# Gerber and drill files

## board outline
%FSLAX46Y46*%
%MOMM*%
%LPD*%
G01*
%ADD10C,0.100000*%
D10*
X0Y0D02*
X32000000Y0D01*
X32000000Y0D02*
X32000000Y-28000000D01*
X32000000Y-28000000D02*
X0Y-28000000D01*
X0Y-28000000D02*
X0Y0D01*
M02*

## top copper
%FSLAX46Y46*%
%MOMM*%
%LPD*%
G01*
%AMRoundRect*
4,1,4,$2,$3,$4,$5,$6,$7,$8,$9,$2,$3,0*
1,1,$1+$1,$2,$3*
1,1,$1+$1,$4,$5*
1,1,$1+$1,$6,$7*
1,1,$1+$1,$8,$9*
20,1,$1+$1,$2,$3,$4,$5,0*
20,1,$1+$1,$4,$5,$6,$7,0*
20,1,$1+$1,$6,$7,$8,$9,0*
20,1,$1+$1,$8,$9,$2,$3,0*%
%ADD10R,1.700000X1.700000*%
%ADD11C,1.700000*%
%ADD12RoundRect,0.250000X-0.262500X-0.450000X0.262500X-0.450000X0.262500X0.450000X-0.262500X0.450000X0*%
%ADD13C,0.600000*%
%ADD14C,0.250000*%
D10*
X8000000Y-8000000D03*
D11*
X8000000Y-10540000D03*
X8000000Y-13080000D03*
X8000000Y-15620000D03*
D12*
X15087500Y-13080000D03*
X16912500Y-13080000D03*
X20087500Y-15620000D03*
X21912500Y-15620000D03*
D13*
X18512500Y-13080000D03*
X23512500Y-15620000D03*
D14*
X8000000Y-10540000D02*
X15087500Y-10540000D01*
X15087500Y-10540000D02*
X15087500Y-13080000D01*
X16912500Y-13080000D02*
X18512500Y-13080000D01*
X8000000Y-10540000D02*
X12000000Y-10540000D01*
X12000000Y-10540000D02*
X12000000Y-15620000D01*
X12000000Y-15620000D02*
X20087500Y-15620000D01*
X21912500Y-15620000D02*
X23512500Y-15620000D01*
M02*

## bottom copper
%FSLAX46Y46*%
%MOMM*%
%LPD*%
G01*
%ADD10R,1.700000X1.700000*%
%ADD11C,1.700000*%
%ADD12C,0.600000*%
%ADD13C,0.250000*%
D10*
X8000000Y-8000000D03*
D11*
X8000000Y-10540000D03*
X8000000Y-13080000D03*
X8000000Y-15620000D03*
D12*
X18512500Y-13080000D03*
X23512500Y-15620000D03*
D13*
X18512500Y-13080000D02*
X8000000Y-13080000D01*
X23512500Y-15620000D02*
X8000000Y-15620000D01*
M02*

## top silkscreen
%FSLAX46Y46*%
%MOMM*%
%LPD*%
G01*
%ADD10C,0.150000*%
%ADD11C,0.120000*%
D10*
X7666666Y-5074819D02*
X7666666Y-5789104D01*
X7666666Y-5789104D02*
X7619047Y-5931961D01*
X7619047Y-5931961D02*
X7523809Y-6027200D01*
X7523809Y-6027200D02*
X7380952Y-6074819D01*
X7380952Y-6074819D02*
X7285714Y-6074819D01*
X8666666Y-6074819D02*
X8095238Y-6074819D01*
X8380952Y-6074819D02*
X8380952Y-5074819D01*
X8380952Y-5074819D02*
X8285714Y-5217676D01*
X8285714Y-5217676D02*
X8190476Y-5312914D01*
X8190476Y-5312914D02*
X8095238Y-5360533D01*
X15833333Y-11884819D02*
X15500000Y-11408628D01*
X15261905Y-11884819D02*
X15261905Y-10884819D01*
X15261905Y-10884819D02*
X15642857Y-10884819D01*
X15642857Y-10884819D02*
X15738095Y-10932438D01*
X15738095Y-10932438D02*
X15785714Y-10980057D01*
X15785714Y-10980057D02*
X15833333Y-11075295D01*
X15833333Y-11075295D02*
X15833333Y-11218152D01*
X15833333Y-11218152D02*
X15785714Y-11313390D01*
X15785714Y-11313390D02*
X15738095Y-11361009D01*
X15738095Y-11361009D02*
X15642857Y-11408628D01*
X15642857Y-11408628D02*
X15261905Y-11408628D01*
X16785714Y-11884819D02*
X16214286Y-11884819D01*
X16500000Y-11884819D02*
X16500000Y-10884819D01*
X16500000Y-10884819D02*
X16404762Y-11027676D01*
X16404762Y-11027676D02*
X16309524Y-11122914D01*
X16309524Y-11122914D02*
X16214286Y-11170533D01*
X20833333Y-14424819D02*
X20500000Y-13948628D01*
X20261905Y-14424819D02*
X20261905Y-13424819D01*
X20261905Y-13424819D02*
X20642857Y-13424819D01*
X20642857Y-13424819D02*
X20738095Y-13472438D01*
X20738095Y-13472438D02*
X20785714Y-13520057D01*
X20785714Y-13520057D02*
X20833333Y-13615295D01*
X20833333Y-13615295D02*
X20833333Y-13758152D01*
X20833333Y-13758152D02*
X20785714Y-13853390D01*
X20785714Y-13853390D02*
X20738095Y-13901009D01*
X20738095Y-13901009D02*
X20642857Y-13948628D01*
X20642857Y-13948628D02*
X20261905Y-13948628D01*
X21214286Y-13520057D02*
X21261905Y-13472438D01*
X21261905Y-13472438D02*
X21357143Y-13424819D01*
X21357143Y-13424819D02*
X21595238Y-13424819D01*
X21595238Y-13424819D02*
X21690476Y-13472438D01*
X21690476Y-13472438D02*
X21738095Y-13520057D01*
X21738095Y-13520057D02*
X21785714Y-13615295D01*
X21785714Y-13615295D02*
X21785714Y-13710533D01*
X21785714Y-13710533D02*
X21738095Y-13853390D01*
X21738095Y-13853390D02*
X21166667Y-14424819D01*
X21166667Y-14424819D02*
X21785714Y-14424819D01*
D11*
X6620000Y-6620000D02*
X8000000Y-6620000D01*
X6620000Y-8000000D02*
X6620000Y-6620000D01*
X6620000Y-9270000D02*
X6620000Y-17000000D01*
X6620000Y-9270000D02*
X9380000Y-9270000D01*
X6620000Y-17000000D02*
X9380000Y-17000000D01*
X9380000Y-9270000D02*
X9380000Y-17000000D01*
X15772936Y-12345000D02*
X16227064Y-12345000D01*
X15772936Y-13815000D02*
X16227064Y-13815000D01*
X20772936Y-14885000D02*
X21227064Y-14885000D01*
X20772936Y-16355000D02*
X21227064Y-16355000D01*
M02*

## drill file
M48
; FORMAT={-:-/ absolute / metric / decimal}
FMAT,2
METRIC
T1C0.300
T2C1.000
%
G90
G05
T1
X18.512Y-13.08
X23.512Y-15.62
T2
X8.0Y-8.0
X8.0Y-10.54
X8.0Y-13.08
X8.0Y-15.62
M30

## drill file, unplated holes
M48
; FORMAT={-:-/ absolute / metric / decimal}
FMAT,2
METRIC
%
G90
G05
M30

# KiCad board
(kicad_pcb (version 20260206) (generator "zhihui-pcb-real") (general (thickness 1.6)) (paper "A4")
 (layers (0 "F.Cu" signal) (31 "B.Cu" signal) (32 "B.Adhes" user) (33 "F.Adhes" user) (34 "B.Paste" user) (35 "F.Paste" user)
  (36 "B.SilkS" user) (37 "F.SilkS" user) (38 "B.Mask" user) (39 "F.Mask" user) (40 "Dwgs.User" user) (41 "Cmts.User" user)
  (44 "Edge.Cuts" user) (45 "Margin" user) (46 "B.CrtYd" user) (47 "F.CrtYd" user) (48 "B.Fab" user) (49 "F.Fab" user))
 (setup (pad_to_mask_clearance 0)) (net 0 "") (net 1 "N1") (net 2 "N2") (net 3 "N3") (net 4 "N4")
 (gr_line (start 0 0) (end 32 0) (stroke (width 0.1) (type default)) (layer "Edge.Cuts"))
 (gr_line (start 32 0) (end 32 28) (stroke (width 0.1) (type default)) (layer "Edge.Cuts"))
 (gr_line (start 32 28) (end 0 28) (stroke (width 0.1) (type default)) (layer "Edge.Cuts"))
 (gr_line (start 0 28) (end 0 0) (stroke (width 0.1) (type default)) (layer "Edge.Cuts"))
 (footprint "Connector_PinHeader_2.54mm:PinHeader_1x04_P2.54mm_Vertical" (layer "F.Cu")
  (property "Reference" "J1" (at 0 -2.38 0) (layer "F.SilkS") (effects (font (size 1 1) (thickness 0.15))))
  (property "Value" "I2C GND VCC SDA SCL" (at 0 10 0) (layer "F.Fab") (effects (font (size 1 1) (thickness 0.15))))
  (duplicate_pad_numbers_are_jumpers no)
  (fp_line (start -1.38 -1.38) (end 0 -1.38) (stroke (width 0.12) (type solid)) (layer "F.SilkS"))
  (fp_line (start -1.38 0) (end -1.38 -1.38) (stroke (width 0.12) (type solid)) (layer "F.SilkS"))
  (fp_line (start -1.38 1.27) (end -1.38 9) (stroke (width 0.12) (type solid)) (layer "F.SilkS"))
  (fp_line (start -1.38 1.27) (end 1.38 1.27) (stroke (width 0.12) (type solid)) (layer "F.SilkS"))
  (fp_line (start -1.38 9) (end 1.38 9) (stroke (width 0.12) (type solid)) (layer "F.SilkS"))
  (fp_line (start 1.38 1.27) (end 1.38 9) (stroke (width 0.12) (type solid)) (layer "F.SilkS"))
  (pad "1" thru_hole rect (at 0 0) (size 1.7 1.7) (drill 1) (layers "*.Cu" "*.Mask") (remove_unused_layers no) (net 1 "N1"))
  (pad "2" thru_hole circle (at 0 2.54) (size 1.7 1.7) (drill 1) (layers "*.Cu" "*.Mask") (remove_unused_layers no) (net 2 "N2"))
  (pad "3" thru_hole circle (at 0 5.08) (size 1.7 1.7) (drill 1) (layers "*.Cu" "*.Mask") (remove_unused_layers no) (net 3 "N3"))
  (pad "4" thru_hole circle (at 0 7.62) (size 1.7 1.7) (drill 1) (layers "*.Cu" "*.Mask") (remove_unused_layers no) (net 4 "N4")) (at 8 8 0))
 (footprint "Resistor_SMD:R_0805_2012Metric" (layer "F.Cu")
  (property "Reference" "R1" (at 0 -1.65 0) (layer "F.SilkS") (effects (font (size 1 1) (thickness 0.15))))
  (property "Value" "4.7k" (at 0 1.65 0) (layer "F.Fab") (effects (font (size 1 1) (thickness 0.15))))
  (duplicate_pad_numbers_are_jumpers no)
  (fp_line (start -0.227064 -0.735) (end 0.227064 -0.735) (stroke (width 0.12) (type solid)) (layer "F.SilkS"))
  (fp_line (start -0.227064 0.735) (end 0.227064 0.735) (stroke (width 0.12) (type solid)) (layer "F.SilkS"))
  (pad "1" smd roundrect (at -0.9125 0) (size 1.025 1.4) (layers "F.Cu" "F.Mask" "F.Paste") (roundrect_rratio 0.243902) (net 2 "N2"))
  (pad "2" smd roundrect (at 0.9125 0) (size 1.025 1.4) (layers "F.Cu" "F.Mask" "F.Paste") (roundrect_rratio 0.243902) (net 3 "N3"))
  (at 16 13.08 0))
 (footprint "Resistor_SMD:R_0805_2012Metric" (layer "F.Cu")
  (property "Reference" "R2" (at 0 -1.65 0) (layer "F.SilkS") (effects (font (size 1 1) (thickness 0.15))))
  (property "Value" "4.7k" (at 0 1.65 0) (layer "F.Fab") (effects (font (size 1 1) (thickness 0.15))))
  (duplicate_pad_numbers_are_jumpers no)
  (fp_line (start -0.227064 -0.735) (end 0.227064 -0.735) (stroke (width 0.12) (type solid)) (layer "F.SilkS"))
  (fp_line (start -0.227064 0.735) (end 0.227064 0.735) (stroke (width 0.12) (type solid)) (layer "F.SilkS"))
  (pad "1" smd roundrect (at -0.9125 0) (size 1.025 1.4) (layers "F.Cu" "F.Mask" "F.Paste") (roundrect_rratio 0.243902) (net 2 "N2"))
  (pad "2" smd roundrect (at 0.9125 0) (size 1.025 1.4) (layers "F.Cu" "F.Mask" "F.Paste") (roundrect_rratio 0.243902) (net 4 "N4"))
  (at 21 15.62 0))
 (segment (start 8 10.54) (end 15.0875 10.54) (width 0.25) (layer "F.Cu") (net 2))
 (segment (start 15.0875 10.54) (end 15.0875 13.08) (width 0.25) (layer "F.Cu") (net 2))
 (segment (start 16.9125 13.08) (end 18.5125 13.08) (width 0.25) (layer "F.Cu") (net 3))
 (segment (start 18.5125 13.08) (end 8 13.08) (width 0.25) (layer "B.Cu") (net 3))
 (segment (start 8 10.54) (end 12 10.54) (width 0.25) (layer "F.Cu") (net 2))
 (segment (start 12 10.54) (end 12 15.62) (width 0.25) (layer "F.Cu") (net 2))
 (segment (start 12 15.62) (end 20.0875 15.62) (width 0.25) (layer "F.Cu") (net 2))
 (segment (start 21.9125 15.62) (end 23.5125 15.62) (width 0.25) (layer "F.Cu") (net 4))
 (segment (start 23.5125 15.62) (end 8 15.62) (width 0.25) (layer "B.Cu") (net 4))
 (via (at 18.5125 13.08) (size 0.6) (drill 0.3) (layers "F.Cu" "B.Cu") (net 3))
 (via (at 23.5125 15.62) (size 0.6) (drill 0.3) (layers "F.Cu" "B.Cu") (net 4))
 (segment (start 8 8) (end 8 10.54) (width 0.25) (layer "F.Cu") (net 2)))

